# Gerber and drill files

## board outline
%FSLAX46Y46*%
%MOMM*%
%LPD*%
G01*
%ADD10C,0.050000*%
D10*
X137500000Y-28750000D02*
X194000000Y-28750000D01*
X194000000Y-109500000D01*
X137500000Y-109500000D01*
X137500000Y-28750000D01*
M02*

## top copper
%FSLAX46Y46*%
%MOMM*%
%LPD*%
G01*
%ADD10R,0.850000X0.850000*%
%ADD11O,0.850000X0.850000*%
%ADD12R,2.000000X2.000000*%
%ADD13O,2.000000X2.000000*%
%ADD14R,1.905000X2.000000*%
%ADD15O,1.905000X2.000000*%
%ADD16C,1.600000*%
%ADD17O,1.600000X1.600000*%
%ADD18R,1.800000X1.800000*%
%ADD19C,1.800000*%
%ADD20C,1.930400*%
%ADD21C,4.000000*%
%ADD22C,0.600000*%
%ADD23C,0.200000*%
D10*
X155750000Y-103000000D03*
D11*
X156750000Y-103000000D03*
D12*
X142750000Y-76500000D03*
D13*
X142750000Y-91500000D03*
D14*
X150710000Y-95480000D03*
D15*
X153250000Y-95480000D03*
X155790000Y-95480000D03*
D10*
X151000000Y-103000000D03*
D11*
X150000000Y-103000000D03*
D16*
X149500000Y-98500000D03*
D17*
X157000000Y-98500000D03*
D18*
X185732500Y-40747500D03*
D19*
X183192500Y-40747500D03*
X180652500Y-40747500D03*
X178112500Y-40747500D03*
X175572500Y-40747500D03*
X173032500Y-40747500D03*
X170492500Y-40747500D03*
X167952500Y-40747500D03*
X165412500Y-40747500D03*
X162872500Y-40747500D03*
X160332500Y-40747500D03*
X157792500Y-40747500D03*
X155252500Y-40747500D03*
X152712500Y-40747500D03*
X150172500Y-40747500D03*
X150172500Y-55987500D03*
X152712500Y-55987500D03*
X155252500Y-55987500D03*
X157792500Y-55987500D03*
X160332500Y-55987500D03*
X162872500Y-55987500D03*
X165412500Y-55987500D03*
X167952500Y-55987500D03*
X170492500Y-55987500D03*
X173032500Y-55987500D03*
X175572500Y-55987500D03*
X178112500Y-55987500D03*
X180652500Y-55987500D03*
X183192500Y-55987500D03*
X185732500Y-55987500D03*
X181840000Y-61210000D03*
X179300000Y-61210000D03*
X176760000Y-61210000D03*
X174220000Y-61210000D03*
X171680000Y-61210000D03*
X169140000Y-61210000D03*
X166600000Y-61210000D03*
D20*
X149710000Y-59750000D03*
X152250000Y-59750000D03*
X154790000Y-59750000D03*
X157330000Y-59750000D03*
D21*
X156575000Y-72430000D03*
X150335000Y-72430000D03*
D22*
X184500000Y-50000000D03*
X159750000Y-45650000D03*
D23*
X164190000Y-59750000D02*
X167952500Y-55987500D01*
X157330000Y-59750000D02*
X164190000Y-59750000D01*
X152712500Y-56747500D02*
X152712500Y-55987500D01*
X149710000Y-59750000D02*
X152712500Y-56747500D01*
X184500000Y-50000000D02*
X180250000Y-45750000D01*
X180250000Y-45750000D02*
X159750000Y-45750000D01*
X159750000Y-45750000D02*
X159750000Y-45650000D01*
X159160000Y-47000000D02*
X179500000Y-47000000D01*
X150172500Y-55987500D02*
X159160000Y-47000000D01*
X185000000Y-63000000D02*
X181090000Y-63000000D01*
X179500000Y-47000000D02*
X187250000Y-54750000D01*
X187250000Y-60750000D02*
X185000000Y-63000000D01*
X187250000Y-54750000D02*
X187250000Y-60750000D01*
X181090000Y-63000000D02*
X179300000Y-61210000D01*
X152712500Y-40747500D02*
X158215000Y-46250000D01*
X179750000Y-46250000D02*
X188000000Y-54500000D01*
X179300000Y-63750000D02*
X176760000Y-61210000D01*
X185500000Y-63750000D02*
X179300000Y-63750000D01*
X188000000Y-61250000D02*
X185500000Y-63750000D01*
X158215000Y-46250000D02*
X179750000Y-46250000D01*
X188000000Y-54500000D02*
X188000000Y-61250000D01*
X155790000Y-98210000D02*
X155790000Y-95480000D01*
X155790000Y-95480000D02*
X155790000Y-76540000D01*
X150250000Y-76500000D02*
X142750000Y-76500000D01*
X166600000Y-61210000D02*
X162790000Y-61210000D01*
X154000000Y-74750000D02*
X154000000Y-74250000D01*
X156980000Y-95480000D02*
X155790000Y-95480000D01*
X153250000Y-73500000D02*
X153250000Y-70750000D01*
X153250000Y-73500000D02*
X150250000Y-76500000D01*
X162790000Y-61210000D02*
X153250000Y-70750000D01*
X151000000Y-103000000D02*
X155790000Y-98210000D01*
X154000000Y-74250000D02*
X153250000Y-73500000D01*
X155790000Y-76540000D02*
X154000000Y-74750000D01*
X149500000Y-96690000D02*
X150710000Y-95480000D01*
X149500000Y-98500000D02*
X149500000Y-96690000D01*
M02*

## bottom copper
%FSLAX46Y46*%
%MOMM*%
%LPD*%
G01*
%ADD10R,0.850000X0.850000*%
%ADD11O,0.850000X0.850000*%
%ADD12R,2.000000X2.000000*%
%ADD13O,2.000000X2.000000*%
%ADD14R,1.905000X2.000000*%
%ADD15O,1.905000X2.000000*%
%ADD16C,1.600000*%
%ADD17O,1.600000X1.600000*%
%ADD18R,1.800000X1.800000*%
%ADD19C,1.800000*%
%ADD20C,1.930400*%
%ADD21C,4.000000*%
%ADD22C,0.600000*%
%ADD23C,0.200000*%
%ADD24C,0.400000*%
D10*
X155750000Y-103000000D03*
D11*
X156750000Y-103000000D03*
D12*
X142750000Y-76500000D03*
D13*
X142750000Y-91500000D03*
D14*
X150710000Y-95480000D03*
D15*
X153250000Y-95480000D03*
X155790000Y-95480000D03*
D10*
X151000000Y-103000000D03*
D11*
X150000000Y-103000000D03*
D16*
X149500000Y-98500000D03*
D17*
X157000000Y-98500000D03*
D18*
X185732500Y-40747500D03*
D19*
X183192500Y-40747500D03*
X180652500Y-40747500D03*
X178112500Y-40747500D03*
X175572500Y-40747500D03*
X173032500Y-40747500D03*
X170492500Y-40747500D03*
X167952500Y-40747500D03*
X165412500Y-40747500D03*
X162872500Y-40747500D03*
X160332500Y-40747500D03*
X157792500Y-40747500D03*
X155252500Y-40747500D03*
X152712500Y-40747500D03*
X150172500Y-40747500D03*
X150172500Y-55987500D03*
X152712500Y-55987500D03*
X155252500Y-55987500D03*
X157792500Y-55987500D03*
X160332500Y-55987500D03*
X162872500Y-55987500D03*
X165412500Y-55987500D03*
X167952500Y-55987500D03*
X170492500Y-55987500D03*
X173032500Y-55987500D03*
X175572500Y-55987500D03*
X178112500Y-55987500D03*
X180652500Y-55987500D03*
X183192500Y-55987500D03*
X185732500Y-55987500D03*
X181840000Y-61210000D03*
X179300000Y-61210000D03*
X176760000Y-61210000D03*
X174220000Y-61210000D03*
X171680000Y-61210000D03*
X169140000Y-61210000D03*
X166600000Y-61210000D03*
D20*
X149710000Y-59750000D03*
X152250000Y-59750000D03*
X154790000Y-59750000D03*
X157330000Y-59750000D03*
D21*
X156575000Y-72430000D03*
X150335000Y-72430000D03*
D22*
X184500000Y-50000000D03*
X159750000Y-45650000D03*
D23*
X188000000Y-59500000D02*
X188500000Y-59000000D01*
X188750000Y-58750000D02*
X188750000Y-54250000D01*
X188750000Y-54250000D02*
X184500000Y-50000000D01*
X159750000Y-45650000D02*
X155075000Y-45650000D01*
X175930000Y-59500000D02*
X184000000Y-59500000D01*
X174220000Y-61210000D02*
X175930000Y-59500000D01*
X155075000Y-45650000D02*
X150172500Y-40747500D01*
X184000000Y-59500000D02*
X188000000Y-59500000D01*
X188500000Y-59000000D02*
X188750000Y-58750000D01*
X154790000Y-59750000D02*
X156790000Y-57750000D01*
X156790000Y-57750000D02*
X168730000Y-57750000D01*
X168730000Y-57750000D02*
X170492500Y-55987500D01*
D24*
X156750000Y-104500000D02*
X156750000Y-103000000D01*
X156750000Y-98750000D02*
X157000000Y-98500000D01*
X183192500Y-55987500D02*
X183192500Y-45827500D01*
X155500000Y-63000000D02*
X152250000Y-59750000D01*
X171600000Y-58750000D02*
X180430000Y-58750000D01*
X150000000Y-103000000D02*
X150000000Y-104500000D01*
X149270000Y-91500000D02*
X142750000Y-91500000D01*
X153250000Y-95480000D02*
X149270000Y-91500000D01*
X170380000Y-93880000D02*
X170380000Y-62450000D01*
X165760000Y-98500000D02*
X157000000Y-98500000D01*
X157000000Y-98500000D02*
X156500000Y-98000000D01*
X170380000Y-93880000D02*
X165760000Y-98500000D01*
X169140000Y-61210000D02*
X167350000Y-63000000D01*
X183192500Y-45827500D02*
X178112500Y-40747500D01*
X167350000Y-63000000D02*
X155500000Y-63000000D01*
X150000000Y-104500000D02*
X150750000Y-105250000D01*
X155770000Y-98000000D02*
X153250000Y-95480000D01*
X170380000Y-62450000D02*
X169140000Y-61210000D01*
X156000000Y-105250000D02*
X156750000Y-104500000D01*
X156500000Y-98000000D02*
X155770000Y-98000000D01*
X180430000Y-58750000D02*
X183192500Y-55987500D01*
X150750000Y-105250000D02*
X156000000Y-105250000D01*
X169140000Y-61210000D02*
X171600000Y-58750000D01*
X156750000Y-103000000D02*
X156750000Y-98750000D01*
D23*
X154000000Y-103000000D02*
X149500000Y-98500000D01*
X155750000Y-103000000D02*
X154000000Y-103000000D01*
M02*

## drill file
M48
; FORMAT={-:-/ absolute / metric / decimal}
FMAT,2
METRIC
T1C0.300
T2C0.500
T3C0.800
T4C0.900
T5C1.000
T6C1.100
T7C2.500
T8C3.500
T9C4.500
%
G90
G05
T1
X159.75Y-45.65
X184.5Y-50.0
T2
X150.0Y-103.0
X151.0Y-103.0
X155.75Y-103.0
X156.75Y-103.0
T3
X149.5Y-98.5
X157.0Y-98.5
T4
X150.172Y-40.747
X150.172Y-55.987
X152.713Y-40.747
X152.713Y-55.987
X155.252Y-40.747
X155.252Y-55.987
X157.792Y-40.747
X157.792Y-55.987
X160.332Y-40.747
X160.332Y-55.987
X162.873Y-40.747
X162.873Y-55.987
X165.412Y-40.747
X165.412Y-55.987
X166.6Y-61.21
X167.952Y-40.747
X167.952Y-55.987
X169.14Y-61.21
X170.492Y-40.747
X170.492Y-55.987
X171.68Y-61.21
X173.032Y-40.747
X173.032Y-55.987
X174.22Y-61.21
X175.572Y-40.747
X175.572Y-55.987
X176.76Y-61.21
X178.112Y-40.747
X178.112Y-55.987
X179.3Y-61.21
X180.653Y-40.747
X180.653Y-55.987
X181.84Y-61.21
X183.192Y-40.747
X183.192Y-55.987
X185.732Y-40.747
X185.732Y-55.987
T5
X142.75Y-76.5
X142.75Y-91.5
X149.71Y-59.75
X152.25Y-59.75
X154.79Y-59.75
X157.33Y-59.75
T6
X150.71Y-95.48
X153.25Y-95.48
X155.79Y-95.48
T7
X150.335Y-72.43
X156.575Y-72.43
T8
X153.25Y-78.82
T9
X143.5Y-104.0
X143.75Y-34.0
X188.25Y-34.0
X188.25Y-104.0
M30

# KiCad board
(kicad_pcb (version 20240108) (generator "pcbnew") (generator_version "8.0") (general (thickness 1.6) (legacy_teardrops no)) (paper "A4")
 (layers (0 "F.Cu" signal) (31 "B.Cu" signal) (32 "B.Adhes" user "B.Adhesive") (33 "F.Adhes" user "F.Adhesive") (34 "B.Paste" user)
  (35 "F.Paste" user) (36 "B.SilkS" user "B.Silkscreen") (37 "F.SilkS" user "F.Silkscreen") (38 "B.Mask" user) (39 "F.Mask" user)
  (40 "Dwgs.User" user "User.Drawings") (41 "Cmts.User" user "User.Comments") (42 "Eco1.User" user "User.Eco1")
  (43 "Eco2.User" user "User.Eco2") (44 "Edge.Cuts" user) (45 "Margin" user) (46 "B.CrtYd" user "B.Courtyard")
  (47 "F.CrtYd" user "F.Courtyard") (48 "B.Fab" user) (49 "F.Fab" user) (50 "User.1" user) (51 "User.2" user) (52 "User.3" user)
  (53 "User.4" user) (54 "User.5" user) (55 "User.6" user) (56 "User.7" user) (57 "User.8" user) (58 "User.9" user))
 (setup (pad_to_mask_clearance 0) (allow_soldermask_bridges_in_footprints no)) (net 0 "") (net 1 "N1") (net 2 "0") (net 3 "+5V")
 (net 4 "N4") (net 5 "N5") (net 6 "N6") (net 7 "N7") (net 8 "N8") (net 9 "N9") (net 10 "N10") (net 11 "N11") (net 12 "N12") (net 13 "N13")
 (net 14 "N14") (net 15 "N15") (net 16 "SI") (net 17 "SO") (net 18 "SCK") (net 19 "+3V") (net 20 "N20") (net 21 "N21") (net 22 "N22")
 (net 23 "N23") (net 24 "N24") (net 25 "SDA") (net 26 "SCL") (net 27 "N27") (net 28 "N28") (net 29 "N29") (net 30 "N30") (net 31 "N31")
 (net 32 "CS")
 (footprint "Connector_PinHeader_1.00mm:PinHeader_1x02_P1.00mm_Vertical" (layer "F.Cu") (at 155.75 103 90)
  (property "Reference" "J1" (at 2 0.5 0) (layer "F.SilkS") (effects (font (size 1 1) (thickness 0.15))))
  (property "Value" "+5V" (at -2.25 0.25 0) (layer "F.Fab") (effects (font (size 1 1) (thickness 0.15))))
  (pad "1" thru_hole rect (at 0 0 90) (size 0.85 0.85) (drill 0.5) (layers "*.Cu" "*.Mask") (remove_unused_layers no) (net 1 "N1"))
  (pad "2" thru_hole oval (at 0 1 90) (size 0.85 0.85) (drill 0.5) (layers "*.Cu" "*.Mask") (remove_unused_layers no) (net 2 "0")))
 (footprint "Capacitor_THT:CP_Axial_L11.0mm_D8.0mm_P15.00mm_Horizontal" (layer "F.Cu") (at 142.75 76.5 -90)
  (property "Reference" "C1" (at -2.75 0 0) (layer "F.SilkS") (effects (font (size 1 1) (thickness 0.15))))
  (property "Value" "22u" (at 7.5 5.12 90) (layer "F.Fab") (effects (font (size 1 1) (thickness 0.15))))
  (pad "1" thru_hole rect (at 0 0 270) (size 2 2) (drill 1) (layers "*.Cu" "*.Mask") (remove_unused_layers no) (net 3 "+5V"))
  (pad "2" thru_hole oval (at 15 0 270) (size 2 2) (drill 1) (layers "*.Cu" "*.Mask") (remove_unused_layers no) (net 2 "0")))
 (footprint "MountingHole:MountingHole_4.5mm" (layer "F.Cu") (at 188.25 104)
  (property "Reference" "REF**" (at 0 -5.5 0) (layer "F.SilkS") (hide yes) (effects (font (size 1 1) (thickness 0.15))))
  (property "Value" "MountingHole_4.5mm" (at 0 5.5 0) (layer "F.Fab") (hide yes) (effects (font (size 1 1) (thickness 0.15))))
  (pad "" np_thru_hole circle (at 0 0) (size 4.5 4.5) (drill 4.5) (layers "*.Cu" "*.Mask")))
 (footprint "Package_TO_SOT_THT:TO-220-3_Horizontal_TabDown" (layer "F.Cu") (at 150.71 95.48)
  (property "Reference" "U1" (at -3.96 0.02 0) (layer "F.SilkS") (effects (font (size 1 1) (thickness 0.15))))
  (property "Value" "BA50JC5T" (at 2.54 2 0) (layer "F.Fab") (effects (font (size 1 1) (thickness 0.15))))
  (pad "" np_thru_hole oval (at 2.54 -16.66) (size 3.5 3.5) (drill 3.5) (layers "*.Cu" "*.Mask"))
  (pad "1" thru_hole rect (at 0 0) (size 1.905 2) (drill 1.1) (layers "*.Cu" "*.Mask") (remove_unused_layers no) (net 1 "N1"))
  (pad "2" thru_hole oval (at 2.54 0) (size 1.905 2) (drill 1.1) (layers "*.Cu" "*.Mask") (remove_unused_layers no) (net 2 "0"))
  (pad "3" thru_hole oval (at 5.08 0) (size 1.905 2) (drill 1.1) (layers "*.Cu" "*.Mask") (remove_unused_layers no) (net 3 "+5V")))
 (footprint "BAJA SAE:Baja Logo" (layer "F.Cu") (at 165.25 32.25)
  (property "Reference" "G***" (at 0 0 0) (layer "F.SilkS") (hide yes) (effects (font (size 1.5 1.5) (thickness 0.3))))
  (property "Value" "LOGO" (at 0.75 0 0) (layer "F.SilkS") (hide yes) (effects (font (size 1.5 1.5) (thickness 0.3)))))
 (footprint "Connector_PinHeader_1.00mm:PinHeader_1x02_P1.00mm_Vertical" (layer "F.Cu") (at 151 103 -90)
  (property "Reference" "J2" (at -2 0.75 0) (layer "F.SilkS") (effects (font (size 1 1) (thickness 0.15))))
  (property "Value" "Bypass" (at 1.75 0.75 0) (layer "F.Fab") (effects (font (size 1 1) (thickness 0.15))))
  (pad "1" thru_hole rect (at 0 0 270) (size 0.85 0.85) (drill 0.5) (layers "*.Cu" "*.Mask") (remove_unused_layers no) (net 3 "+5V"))
  (pad "2" thru_hole oval (at 0 1 270) (size 0.85 0.85) (drill 0.5) (layers "*.Cu" "*.Mask") (remove_unused_layers no) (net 2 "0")))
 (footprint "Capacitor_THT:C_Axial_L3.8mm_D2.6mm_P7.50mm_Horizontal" (layer "F.Cu") (at 149.5 98.5)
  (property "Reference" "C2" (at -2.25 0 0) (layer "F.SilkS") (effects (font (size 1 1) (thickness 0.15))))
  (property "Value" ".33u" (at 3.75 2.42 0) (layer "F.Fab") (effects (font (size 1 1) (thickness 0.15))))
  (pad "1" thru_hole circle (at 0 0) (size 1.6 1.6) (drill 0.8) (layers "*.Cu" "*.Mask") (remove_unused_layers no) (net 1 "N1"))
  (pad "2" thru_hole oval (at 7.5 0) (size 1.6 1.6) (drill 0.8) (layers "*.Cu" "*.Mask") (remove_unused_layers no) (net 2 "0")))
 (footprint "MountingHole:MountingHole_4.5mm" (layer "F.Cu") (at 143.5 104)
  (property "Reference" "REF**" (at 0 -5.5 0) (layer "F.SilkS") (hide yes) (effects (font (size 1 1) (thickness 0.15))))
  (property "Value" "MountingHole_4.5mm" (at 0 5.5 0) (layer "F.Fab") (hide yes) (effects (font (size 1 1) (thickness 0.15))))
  (pad "" np_thru_hole circle (at 0 0) (size 4.5 4.5) (drill 4.5) (layers "*.Cu" "*.Mask")))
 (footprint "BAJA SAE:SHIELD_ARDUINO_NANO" (layer "F.Cu") (at 167.9525 48.3675 -90)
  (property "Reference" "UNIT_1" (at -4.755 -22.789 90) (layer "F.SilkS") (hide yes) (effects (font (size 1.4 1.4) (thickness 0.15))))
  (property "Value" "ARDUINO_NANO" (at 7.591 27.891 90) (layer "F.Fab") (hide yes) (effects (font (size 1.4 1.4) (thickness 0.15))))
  (pad "1" thru_hole rect (at -7.62 -17.78 270) (size 1.8 1.8) (drill 0.9) (layers "*.Cu" "*.Mask") (remove_unused_layers no) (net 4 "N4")
   (solder_mask_margin 0.102))
  (pad "2" thru_hole circle (at -7.62 -15.24 270) (size 1.8 1.8) (drill 0.9) (layers "*.Cu" "*.Mask") (remove_unused_layers no) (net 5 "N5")
   (solder_mask_margin 0.102))
  (pad "3" thru_hole circle (at -7.62 -12.7 270) (size 1.8 1.8) (drill 0.9) (layers "*.Cu" "*.Mask") (remove_unused_layers no) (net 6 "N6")
   (solder_mask_margin 0.102))
  (pad "4" thru_hole circle (at -7.62 -10.16 270) (size 1.8 1.8) (drill 0.9) (layers "*.Cu" "*.Mask") (remove_unused_layers no) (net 2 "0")
   (solder_mask_margin 0.102))
  (pad "5" thru_hole circle (at -7.62 -7.62 270) (size 1.8 1.8) (drill 0.9) (layers "*.Cu" "*.Mask") (remove_unused_layers no) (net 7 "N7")
   (solder_mask_margin 0.102))
  (pad "6" thru_hole circle (at -7.62 -5.08 270) (size 1.8 1.8) (drill 0.9) (layers "*.Cu" "*.Mask") (remove_unused_layers no) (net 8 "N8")
   (solder_mask_margin 0.102))
  (pad "7" thru_hole circle (at -7.62 -2.54 270) (size 1.8 1.8) (drill 0.9) (layers "*.Cu" "*.Mask") (remove_unused_layers no) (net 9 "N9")
   (solder_mask_margin 0.102))
  (pad "8" thru_hole circle (at -7.62 0 270) (size 1.8 1.8) (drill 0.9) (layers "*.Cu" "*.Mask") (remove_unused_layers no) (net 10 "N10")
   (solder_mask_margin 0.102))
  (pad "9" thru_hole circle (at -7.62 2.54 270) (size 1.8 1.8) (drill 0.9) (layers "*.Cu" "*.Mask") (remove_unused_layers no) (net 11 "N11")
   (solder_mask_margin 0.102))
  (pad "10" thru_hole circle (at -7.62 5.08 270) (size 1.8 1.8) (drill 0.9) (layers "*.Cu" "*.Mask") (remove_unused_layers no)
   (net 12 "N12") (solder_mask_margin 0.102))
  (pad "11" thru_hole circle (at -7.62 7.62 270) (size 1.8 1.8) (drill 0.9) (layers "*.Cu" "*.Mask") (remove_unused_layers no)
   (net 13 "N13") (solder_mask_margin 0.102))
  (pad "12" thru_hole circle (at -7.62 10.16 270) (size 1.8 1.8) (drill 0.9) (layers "*.Cu" "*.Mask") (remove_unused_layers no)
   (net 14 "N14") (solder_mask_margin 0.102))
  (pad "13" thru_hole circle (at -7.62 12.7 270) (size 1.8 1.8) (drill 0.9) (layers "*.Cu" "*.Mask") (remove_unused_layers no)
   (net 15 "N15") (solder_mask_margin 0.102))
  (pad "14" thru_hole circle (at -7.62 15.24 270) (size 1.8 1.8) (drill 0.9) (layers "*.Cu" "*.Mask") (remove_unused_layers no)
   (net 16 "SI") (solder_mask_margin 0.102))
  (pad "15" thru_hole circle (at -7.62 17.78 270) (size 1.8 1.8) (drill 0.9) (layers "*.Cu" "*.Mask") (remove_unused_layers no)
   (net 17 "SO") (solder_mask_margin 0.102))
  (pad "16" thru_hole circle (at 7.62 17.78 270) (size 1.8 1.8) (drill 0.9) (layers "*.Cu" "*.Mask") (remove_unused_layers no)
   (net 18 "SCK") (solder_mask_margin 0.102))
  (pad "17" thru_hole circle (at 7.62 15.24 270) (size 1.8 1.8) (drill 0.9) (layers "*.Cu" "*.Mask") (remove_unused_layers no)
   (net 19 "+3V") (solder_mask_margin 0.102))
  (pad "18" thru_hole circle (at 7.62 12.7 270) (size 1.8 1.8) (drill 0.9) (layers "*.Cu" "*.Mask") (remove_unused_layers no) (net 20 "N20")
   (solder_mask_margin 0.102))
  (pad "19" thru_hole circle (at 7.62 10.16 270) (size 1.8 1.8) (drill 0.9) (layers "*.Cu" "*.Mask") (remove_unused_layers no)
   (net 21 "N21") (solder_mask_margin 0.102))
  (pad "20" thru_hole circle (at 7.62 7.62 270) (size 1.8 1.8) (drill 0.9) (layers "*.Cu" "*.Mask") (remove_unused_layers no) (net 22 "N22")
   (solder_mask_margin 0.102))
  (pad "21" thru_hole circle (at 7.62 5.08 270) (size 1.8 1.8) (drill 0.9) (layers "*.Cu" "*.Mask") (remove_unused_layers no) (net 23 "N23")
   (solder_mask_margin 0.102))
  (pad "22" thru_hole circle (at 7.62 2.54 270) (size 1.8 1.8) (drill 0.9) (layers "*.Cu" "*.Mask") (remove_unused_layers no) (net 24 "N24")
   (solder_mask_margin 0.102))
  (pad "23" thru_hole circle (at 7.62 0 270) (size 1.8 1.8) (drill 0.9) (layers "*.Cu" "*.Mask") (remove_unused_layers no) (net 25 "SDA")
   (solder_mask_margin 0.102))
  (pad "24" thru_hole circle (at 7.62 -2.54 270) (size 1.8 1.8) (drill 0.9) (layers "*.Cu" "*.Mask") (remove_unused_layers no)
   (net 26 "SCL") (solder_mask_margin 0.102))
  (pad "25" thru_hole circle (at 7.62 -5.08 270) (size 1.8 1.8) (drill 0.9) (layers "*.Cu" "*.Mask") (remove_unused_layers no)
   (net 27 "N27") (solder_mask_margin 0.102))
  (pad "26" thru_hole circle (at 7.62 -7.62 270) (size 1.8 1.8) (drill 0.9) (layers "*.Cu" "*.Mask") (remove_unused_layers no)
   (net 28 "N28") (solder_mask_margin 0.102))
  (pad "27" thru_hole circle (at 7.62 -10.16 270) (size 1.8 1.8) (drill 0.9) (layers "*.Cu" "*.Mask") (remove_unused_layers no)
   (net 3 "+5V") (solder_mask_margin 0.102))
  (pad "28" thru_hole circle (at 7.62 -12.7 270) (size 1.8 1.8) (drill 0.9) (layers "*.Cu" "*.Mask") (remove_unused_layers no)
   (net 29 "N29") (solder_mask_margin 0.102))
  (pad "29" thru_hole circle (at 7.62 -15.24 270) (size 1.8 1.8) (drill 0.9) (layers "*.Cu" "*.Mask") (remove_unused_layers no) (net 2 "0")
   (solder_mask_margin 0.102))
  (pad "30" thru_hole circle (at 7.62 -17.78 270) (size 1.8 1.8) (drill 0.9) (layers "*.Cu" "*.Mask") (remove_unused_layers no)
   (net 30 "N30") (solder_mask_margin 0.102)))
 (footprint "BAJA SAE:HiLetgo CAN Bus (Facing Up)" (layer "F.Cu") (at 174.25 79.25 -90)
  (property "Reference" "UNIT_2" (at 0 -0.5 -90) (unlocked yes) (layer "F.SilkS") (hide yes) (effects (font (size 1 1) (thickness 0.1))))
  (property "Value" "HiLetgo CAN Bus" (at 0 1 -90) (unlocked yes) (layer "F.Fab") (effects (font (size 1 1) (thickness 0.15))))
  (pad "1" thru_hole circle (at -18.04 -7.59 270) (size 1.8 1.8) (drill 0.9) (layers "*.Cu" "*.Mask") (remove_unused_layers no)
   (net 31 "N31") (solder_mask_margin 0.102))
  (pad "2" thru_hole circle (at -18.04 -5.05 270) (size 1.8 1.8) (drill 0.9) (layers "*.Cu" "*.Mask") (remove_unused_layers no)
   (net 18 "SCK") (solder_mask_margin 0.102))
  (pad "3" thru_hole circle (at -18.04 -2.51 270) (size 1.8 1.8) (drill 0.9) (layers "*.Cu" "*.Mask") (remove_unused_layers no)
   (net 16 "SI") (solder_mask_margin 0.102))
  (pad "4" thru_hole circle (at -18.04 0.03 270) (size 1.8 1.8) (drill 0.9) (layers "*.Cu" "*.Mask") (remove_unused_layers no) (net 17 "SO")
   (solder_mask_margin 0.102))
  (pad "5" thru_hole circle (at -18.04 2.57 270) (size 1.8 1.8) (drill 0.9) (layers "*.Cu" "*.Mask") (remove_unused_layers no) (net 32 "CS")
   (solder_mask_margin 0.102))
  (pad "6" thru_hole circle (at -18.04 5.11 270) (size 1.8 1.8) (drill 0.9) (layers "*.Cu" "*.Mask") (remove_unused_layers no) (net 2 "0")
   (solder_mask_margin 0.102))
  (pad "7" thru_hole circle (at -18.04 7.65 270) (size 1.8 1.8) (drill 0.9) (layers "*.Cu" "*.Mask") (remove_unused_layers no) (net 3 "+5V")
   (solder_mask_margin 0.102)))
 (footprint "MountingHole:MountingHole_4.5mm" (layer "F.Cu") (at 143.75 34)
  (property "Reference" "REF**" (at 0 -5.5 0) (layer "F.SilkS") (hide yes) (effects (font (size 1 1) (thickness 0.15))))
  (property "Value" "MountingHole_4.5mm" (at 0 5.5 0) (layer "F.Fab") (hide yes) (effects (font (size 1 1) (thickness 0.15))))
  (pad "" np_thru_hole circle (at 0 0) (size 4.5 4.5) (drill 4.5) (layers "*.Cu" "*.Mask")))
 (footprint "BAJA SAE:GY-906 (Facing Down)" (layer "F.Cu") (at 153.455 68.26)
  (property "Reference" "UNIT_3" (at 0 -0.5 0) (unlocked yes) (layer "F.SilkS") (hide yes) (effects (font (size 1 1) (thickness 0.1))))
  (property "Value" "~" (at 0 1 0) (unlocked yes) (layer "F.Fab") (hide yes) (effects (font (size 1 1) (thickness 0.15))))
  (pad "1" thru_hole circle (at -3.745 -8.51) (size 1.9304 1.9304) (drill 1) (layers "*.Cu" "*.Mask") (remove_unused_layers no)
   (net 19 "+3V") (solder_mask_margin 0.102))
  (pad "2" thru_hole circle (at -1.205 -8.51) (size 1.9304 1.9304) (drill 1) (layers "*.Cu" "*.Mask") (remove_unused_layers no) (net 2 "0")
   (solder_mask_margin 0.102))
  (pad "3" thru_hole circle (at 1.335 -8.51) (size 1.9304 1.9304) (drill 1) (layers "*.Cu" "*.Mask") (remove_unused_layers no)
   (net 26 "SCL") (solder_mask_margin 0.102))
  (pad "4" thru_hole circle (at 3.875 -8.51) (size 1.9304 1.9304) (drill 1) (layers "*.Cu" "*.Mask") (remove_unused_layers no)
   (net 25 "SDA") (solder_mask_margin 0.102))
  (pad "SH3" thru_hole circle (at 3.12 4.17) (size 4 4) (drill 2.5) (layers "*.Cu" "*.Mask") (remove_unused_layers no)
   (solder_mask_margin 0.102))
  (pad "SH4" thru_hole circle (at -3.12 4.17) (size 4 4) (drill 2.5) (layers "*.Cu" "*.Mask") (remove_unused_layers no)
   (solder_mask_margin 0.102)))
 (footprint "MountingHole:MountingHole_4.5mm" (layer "F.Cu") (at 188.25 34)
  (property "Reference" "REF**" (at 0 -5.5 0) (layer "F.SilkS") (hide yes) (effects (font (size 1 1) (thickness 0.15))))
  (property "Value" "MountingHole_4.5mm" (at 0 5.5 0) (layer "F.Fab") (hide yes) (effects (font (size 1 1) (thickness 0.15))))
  (pad "" np_thru_hole circle (at 0 0) (size 4.5 4.5) (drill 4.5) (layers "*.Cu" "*.Mask")))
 (gr_rect (start 137.5 28.75) (end 194 109.5) (stroke (width 0.05) (type default)) (fill none) (layer "Edge.Cuts"))
 (segment (start 164.19 59.75) (end 167.9525 55.9875) (width 0.2) (layer "F.Cu") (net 25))
 (segment (start 157.33 59.75) (end 164.19 59.75) (width 0.2) (layer "F.Cu") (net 25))
 (segment (start 152.7125 56.7475) (end 152.7125 55.9875) (width 0.2) (layer "F.Cu") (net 19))
 (segment (start 149.71 59.75) (end 152.7125 56.7475) (width 0.2) (layer "F.Cu") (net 19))
 (segment (start 184.5 50) (end 180.25 45.75) (width 0.2) (layer "F.Cu") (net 17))
 (segment (start 180.25 45.75) (end 159.75 45.75) (width 0.2) (layer "F.Cu") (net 17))
 (segment (start 159.75 45.75) (end 159.75 45.65) (width 0.2) (layer "F.Cu") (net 17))
 (via (at 184.5 50) (size 0.6) (drill 0.3) (layers "F.Cu" "B.Cu") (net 17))
 (via (at 159.75 45.65) (size 0.6) (drill 0.3) (layers "F.Cu" "B.Cu") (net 17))
 (segment (start 188 59.5) (end 188.5 59) (width 0.2) (layer "B.Cu") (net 17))
 (segment (start 188.75 58.75) (end 188.75 54.25) (width 0.2) (layer "B.Cu") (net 17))
 (segment (start 188.75 54.25) (end 184.5 50) (width 0.2) (layer "B.Cu") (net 17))
 (segment (start 159.75 45.65) (end 155.075 45.65) (width 0.2) (layer "B.Cu") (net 17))
 (segment (start 175.93 59.5) (end 184 59.5) (width 0.2) (layer "B.Cu") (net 17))
 (segment (start 174.22 61.21) (end 175.93 59.5) (width 0.2) (layer "B.Cu") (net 17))
 (segment (start 155.075 45.65) (end 150.1725 40.7475) (width 0.2) (layer "B.Cu") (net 17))
 (segment (start 184 59.5) (end 188 59.5) (width 0.2) (layer "B.Cu") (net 17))
 (segment (start 188.5 59) (end 188.75 58.75) (width 0.2) (layer "B.Cu") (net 17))
 (segment (start 159.16 47) (end 179.5 47) (width 0.2) (layer "F.Cu") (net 18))
 (segment (start 150.1725 55.9875) (end 159.16 47) (width 0.2) (layer "F.Cu") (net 18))
 (segment (start 185 63) (end 181.09 63) (width 0.2) (layer "F.Cu") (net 18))
 (segment (start 179.5 47) (end 187.25 54.75) (width 0.2) (layer "F.Cu") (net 18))
 (segment (start 187.25 60.75) (end 185 63) (width 0.2) (layer "F.Cu") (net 18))
 (segment (start 187.25 54.75) (end 187.25 60.75) (width 0.2) (layer "F.Cu") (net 18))
 (segment (start 181.09 63) (end 179.3 61.21) (width 0.2) (layer "F.Cu") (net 18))
 (segment (start 152.7125 40.7475) (end 158.215 46.25) (width 0.2) (layer "F.Cu") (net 16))
 (segment (start 179.75 46.25) (end 188 54.5) (width 0.2) (layer "F.Cu") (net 16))
 (segment (start 179.3 63.75) (end 176.76 61.21) (width 0.2) (layer "F.Cu") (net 16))
 (segment (start 185.5 63.75) (end 179.3 63.75) (width 0.2) (layer "F.Cu") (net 16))
 (segment (start 188 61.25) (end 185.5 63.75) (width 0.2) (layer "F.Cu") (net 16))
 (segment (start 158.215 46.25) (end 179.75 46.25) (width 0.2) (layer "F.Cu") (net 16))
 (segment (start 188 54.5) (end 188 61.25) (width 0.2) (layer "F.Cu") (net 16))
 (segment (start 154.79 59.75) (end 156.79 57.75) (width 0.2) (layer "B.Cu") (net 26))
 (segment (start 156.79 57.75) (end 168.73 57.75) (width 0.2) (layer "B.Cu") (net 26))
 (segment (start 168.73 57.75) (end 170.4925 55.9875) (width 0.2) (layer "B.Cu") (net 26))
 (segment (start 155.79 98.21) (end 155.79 95.48) (width 0.2) (layer "F.Cu") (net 3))
 (segment (start 155.79 95.48) (end 155.79 76.54) (width 0.2) (layer "F.Cu") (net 3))
 (segment (start 150.25 76.5) (end 142.75 76.5) (width 0.2) (layer "F.Cu") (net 3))
 (segment (start 166.6 61.21) (end 162.79 61.21) (width 0.2) (layer "F.Cu") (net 3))
 (segment (start 154 74.75) (end 154 74.25) (width 0.2) (layer "F.Cu") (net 3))
 (segment (start 156.98 95.48) (end 155.79 95.48) (width 0.2) (layer "F.Cu") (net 3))
 (segment (start 153.25 73.5) (end 153.25 70.75) (width 0.2) (layer "F.Cu") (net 3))
 (segment (start 153.25 73.5) (end 150.25 76.5) (width 0.2) (layer "F.Cu") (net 3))
 (segment (start 162.79 61.21) (end 153.25 70.75) (width 0.2) (layer "F.Cu") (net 3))
 (segment (start 151 103) (end 155.79 98.21) (width 0.2) (layer "F.Cu") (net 3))
 (segment (start 154 74.25) (end 153.25 73.5) (width 0.2) (layer "F.Cu") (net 3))
 (segment (start 155.79 76.54) (end 154 74.75) (width 0.2) (layer "F.Cu") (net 3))
 (segment (start 156.75 104.5) (end 156.75 103) (width 0.4) (layer "B.Cu") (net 2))
 (segment (start 156.75 98.75) (end 157 98.5) (width 0.4) (layer "B.Cu") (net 2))
 (segment (start 183.1925 55.9875) (end 183.1925 45.8275) (width 0.4) (layer "B.Cu") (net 2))
 (segment (start 155.5 63) (end 152.25 59.75) (width 0.4) (layer "B.Cu") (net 2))
 (segment (start 171.6 58.75) (end 180.43 58.75) (width 0.4) (layer "B.Cu") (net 2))
 (segment (start 150 103) (end 150 104.5) (width 0.4) (layer "B.Cu") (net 2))
 (segment (start 149.27 91.5) (end 142.75 91.5) (width 0.4) (layer "B.Cu") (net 2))
 (segment (start 153.25 95.48) (end 149.27 91.5) (width 0.4) (layer "B.Cu") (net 2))
 (segment (start 170.38 93.88) (end 170.38 62.45) (width 0.4) (layer "B.Cu") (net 2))
 (segment (start 165.76 98.5) (end 157 98.5) (width 0.4) (layer "B.Cu") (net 2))
 (segment (start 157 98.5) (end 156.5 98) (width 0.4) (layer "B.Cu") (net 2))
 (segment (start 170.38 93.88) (end 165.76 98.5) (width 0.4) (layer "B.Cu") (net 2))
 (segment (start 169.14 61.21) (end 167.35 63) (width 0.4) (layer "B.Cu") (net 2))
 (segment (start 183.1925 45.8275) (end 178.1125 40.7475) (width 0.4) (layer "B.Cu") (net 2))
 (segment (start 167.35 63) (end 155.5 63) (width 0.4) (layer "B.Cu") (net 2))
 (segment (start 150 104.5) (end 150.75 105.25) (width 0.4) (layer "B.Cu") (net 2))
 (segment (start 155.77 98) (end 153.25 95.48) (width 0.4) (layer "B.Cu") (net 2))
 (segment (start 170.38 62.45) (end 169.14 61.21) (width 0.4) (layer "B.Cu") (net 2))
 (segment (start 156 105.25) (end 156.75 104.5) (width 0.4) (layer "B.Cu") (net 2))
 (segment (start 156.5 98) (end 155.77 98) (width 0.4) (layer "B.Cu") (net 2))
 (segment (start 180.43 58.75) (end 183.1925 55.9875) (width 0.4) (layer "B.Cu") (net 2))
 (segment (start 150.75 105.25) (end 156 105.25) (width 0.4) (layer "B.Cu") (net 2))
 (segment (start 169.14 61.21) (end 171.6 58.75) (width 0.4) (layer "B.Cu") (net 2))
 (segment (start 156.75 103) (end 156.75 98.75) (width 0.4) (layer "B.Cu") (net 2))
 (segment (start 149.5 96.69) (end 150.71 95.48) (width 0.2) (layer "F.Cu") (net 1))
 (segment (start 149.5 98.5) (end 149.5 96.69) (width 0.2) (layer "F.Cu") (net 1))
 (segment (start 154 103) (end 149.5 98.5) (width 0.2) (layer "B.Cu") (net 1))
 (segment (start 155.75 103) (end 154 103) (width 0.2) (layer "B.Cu") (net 1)))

